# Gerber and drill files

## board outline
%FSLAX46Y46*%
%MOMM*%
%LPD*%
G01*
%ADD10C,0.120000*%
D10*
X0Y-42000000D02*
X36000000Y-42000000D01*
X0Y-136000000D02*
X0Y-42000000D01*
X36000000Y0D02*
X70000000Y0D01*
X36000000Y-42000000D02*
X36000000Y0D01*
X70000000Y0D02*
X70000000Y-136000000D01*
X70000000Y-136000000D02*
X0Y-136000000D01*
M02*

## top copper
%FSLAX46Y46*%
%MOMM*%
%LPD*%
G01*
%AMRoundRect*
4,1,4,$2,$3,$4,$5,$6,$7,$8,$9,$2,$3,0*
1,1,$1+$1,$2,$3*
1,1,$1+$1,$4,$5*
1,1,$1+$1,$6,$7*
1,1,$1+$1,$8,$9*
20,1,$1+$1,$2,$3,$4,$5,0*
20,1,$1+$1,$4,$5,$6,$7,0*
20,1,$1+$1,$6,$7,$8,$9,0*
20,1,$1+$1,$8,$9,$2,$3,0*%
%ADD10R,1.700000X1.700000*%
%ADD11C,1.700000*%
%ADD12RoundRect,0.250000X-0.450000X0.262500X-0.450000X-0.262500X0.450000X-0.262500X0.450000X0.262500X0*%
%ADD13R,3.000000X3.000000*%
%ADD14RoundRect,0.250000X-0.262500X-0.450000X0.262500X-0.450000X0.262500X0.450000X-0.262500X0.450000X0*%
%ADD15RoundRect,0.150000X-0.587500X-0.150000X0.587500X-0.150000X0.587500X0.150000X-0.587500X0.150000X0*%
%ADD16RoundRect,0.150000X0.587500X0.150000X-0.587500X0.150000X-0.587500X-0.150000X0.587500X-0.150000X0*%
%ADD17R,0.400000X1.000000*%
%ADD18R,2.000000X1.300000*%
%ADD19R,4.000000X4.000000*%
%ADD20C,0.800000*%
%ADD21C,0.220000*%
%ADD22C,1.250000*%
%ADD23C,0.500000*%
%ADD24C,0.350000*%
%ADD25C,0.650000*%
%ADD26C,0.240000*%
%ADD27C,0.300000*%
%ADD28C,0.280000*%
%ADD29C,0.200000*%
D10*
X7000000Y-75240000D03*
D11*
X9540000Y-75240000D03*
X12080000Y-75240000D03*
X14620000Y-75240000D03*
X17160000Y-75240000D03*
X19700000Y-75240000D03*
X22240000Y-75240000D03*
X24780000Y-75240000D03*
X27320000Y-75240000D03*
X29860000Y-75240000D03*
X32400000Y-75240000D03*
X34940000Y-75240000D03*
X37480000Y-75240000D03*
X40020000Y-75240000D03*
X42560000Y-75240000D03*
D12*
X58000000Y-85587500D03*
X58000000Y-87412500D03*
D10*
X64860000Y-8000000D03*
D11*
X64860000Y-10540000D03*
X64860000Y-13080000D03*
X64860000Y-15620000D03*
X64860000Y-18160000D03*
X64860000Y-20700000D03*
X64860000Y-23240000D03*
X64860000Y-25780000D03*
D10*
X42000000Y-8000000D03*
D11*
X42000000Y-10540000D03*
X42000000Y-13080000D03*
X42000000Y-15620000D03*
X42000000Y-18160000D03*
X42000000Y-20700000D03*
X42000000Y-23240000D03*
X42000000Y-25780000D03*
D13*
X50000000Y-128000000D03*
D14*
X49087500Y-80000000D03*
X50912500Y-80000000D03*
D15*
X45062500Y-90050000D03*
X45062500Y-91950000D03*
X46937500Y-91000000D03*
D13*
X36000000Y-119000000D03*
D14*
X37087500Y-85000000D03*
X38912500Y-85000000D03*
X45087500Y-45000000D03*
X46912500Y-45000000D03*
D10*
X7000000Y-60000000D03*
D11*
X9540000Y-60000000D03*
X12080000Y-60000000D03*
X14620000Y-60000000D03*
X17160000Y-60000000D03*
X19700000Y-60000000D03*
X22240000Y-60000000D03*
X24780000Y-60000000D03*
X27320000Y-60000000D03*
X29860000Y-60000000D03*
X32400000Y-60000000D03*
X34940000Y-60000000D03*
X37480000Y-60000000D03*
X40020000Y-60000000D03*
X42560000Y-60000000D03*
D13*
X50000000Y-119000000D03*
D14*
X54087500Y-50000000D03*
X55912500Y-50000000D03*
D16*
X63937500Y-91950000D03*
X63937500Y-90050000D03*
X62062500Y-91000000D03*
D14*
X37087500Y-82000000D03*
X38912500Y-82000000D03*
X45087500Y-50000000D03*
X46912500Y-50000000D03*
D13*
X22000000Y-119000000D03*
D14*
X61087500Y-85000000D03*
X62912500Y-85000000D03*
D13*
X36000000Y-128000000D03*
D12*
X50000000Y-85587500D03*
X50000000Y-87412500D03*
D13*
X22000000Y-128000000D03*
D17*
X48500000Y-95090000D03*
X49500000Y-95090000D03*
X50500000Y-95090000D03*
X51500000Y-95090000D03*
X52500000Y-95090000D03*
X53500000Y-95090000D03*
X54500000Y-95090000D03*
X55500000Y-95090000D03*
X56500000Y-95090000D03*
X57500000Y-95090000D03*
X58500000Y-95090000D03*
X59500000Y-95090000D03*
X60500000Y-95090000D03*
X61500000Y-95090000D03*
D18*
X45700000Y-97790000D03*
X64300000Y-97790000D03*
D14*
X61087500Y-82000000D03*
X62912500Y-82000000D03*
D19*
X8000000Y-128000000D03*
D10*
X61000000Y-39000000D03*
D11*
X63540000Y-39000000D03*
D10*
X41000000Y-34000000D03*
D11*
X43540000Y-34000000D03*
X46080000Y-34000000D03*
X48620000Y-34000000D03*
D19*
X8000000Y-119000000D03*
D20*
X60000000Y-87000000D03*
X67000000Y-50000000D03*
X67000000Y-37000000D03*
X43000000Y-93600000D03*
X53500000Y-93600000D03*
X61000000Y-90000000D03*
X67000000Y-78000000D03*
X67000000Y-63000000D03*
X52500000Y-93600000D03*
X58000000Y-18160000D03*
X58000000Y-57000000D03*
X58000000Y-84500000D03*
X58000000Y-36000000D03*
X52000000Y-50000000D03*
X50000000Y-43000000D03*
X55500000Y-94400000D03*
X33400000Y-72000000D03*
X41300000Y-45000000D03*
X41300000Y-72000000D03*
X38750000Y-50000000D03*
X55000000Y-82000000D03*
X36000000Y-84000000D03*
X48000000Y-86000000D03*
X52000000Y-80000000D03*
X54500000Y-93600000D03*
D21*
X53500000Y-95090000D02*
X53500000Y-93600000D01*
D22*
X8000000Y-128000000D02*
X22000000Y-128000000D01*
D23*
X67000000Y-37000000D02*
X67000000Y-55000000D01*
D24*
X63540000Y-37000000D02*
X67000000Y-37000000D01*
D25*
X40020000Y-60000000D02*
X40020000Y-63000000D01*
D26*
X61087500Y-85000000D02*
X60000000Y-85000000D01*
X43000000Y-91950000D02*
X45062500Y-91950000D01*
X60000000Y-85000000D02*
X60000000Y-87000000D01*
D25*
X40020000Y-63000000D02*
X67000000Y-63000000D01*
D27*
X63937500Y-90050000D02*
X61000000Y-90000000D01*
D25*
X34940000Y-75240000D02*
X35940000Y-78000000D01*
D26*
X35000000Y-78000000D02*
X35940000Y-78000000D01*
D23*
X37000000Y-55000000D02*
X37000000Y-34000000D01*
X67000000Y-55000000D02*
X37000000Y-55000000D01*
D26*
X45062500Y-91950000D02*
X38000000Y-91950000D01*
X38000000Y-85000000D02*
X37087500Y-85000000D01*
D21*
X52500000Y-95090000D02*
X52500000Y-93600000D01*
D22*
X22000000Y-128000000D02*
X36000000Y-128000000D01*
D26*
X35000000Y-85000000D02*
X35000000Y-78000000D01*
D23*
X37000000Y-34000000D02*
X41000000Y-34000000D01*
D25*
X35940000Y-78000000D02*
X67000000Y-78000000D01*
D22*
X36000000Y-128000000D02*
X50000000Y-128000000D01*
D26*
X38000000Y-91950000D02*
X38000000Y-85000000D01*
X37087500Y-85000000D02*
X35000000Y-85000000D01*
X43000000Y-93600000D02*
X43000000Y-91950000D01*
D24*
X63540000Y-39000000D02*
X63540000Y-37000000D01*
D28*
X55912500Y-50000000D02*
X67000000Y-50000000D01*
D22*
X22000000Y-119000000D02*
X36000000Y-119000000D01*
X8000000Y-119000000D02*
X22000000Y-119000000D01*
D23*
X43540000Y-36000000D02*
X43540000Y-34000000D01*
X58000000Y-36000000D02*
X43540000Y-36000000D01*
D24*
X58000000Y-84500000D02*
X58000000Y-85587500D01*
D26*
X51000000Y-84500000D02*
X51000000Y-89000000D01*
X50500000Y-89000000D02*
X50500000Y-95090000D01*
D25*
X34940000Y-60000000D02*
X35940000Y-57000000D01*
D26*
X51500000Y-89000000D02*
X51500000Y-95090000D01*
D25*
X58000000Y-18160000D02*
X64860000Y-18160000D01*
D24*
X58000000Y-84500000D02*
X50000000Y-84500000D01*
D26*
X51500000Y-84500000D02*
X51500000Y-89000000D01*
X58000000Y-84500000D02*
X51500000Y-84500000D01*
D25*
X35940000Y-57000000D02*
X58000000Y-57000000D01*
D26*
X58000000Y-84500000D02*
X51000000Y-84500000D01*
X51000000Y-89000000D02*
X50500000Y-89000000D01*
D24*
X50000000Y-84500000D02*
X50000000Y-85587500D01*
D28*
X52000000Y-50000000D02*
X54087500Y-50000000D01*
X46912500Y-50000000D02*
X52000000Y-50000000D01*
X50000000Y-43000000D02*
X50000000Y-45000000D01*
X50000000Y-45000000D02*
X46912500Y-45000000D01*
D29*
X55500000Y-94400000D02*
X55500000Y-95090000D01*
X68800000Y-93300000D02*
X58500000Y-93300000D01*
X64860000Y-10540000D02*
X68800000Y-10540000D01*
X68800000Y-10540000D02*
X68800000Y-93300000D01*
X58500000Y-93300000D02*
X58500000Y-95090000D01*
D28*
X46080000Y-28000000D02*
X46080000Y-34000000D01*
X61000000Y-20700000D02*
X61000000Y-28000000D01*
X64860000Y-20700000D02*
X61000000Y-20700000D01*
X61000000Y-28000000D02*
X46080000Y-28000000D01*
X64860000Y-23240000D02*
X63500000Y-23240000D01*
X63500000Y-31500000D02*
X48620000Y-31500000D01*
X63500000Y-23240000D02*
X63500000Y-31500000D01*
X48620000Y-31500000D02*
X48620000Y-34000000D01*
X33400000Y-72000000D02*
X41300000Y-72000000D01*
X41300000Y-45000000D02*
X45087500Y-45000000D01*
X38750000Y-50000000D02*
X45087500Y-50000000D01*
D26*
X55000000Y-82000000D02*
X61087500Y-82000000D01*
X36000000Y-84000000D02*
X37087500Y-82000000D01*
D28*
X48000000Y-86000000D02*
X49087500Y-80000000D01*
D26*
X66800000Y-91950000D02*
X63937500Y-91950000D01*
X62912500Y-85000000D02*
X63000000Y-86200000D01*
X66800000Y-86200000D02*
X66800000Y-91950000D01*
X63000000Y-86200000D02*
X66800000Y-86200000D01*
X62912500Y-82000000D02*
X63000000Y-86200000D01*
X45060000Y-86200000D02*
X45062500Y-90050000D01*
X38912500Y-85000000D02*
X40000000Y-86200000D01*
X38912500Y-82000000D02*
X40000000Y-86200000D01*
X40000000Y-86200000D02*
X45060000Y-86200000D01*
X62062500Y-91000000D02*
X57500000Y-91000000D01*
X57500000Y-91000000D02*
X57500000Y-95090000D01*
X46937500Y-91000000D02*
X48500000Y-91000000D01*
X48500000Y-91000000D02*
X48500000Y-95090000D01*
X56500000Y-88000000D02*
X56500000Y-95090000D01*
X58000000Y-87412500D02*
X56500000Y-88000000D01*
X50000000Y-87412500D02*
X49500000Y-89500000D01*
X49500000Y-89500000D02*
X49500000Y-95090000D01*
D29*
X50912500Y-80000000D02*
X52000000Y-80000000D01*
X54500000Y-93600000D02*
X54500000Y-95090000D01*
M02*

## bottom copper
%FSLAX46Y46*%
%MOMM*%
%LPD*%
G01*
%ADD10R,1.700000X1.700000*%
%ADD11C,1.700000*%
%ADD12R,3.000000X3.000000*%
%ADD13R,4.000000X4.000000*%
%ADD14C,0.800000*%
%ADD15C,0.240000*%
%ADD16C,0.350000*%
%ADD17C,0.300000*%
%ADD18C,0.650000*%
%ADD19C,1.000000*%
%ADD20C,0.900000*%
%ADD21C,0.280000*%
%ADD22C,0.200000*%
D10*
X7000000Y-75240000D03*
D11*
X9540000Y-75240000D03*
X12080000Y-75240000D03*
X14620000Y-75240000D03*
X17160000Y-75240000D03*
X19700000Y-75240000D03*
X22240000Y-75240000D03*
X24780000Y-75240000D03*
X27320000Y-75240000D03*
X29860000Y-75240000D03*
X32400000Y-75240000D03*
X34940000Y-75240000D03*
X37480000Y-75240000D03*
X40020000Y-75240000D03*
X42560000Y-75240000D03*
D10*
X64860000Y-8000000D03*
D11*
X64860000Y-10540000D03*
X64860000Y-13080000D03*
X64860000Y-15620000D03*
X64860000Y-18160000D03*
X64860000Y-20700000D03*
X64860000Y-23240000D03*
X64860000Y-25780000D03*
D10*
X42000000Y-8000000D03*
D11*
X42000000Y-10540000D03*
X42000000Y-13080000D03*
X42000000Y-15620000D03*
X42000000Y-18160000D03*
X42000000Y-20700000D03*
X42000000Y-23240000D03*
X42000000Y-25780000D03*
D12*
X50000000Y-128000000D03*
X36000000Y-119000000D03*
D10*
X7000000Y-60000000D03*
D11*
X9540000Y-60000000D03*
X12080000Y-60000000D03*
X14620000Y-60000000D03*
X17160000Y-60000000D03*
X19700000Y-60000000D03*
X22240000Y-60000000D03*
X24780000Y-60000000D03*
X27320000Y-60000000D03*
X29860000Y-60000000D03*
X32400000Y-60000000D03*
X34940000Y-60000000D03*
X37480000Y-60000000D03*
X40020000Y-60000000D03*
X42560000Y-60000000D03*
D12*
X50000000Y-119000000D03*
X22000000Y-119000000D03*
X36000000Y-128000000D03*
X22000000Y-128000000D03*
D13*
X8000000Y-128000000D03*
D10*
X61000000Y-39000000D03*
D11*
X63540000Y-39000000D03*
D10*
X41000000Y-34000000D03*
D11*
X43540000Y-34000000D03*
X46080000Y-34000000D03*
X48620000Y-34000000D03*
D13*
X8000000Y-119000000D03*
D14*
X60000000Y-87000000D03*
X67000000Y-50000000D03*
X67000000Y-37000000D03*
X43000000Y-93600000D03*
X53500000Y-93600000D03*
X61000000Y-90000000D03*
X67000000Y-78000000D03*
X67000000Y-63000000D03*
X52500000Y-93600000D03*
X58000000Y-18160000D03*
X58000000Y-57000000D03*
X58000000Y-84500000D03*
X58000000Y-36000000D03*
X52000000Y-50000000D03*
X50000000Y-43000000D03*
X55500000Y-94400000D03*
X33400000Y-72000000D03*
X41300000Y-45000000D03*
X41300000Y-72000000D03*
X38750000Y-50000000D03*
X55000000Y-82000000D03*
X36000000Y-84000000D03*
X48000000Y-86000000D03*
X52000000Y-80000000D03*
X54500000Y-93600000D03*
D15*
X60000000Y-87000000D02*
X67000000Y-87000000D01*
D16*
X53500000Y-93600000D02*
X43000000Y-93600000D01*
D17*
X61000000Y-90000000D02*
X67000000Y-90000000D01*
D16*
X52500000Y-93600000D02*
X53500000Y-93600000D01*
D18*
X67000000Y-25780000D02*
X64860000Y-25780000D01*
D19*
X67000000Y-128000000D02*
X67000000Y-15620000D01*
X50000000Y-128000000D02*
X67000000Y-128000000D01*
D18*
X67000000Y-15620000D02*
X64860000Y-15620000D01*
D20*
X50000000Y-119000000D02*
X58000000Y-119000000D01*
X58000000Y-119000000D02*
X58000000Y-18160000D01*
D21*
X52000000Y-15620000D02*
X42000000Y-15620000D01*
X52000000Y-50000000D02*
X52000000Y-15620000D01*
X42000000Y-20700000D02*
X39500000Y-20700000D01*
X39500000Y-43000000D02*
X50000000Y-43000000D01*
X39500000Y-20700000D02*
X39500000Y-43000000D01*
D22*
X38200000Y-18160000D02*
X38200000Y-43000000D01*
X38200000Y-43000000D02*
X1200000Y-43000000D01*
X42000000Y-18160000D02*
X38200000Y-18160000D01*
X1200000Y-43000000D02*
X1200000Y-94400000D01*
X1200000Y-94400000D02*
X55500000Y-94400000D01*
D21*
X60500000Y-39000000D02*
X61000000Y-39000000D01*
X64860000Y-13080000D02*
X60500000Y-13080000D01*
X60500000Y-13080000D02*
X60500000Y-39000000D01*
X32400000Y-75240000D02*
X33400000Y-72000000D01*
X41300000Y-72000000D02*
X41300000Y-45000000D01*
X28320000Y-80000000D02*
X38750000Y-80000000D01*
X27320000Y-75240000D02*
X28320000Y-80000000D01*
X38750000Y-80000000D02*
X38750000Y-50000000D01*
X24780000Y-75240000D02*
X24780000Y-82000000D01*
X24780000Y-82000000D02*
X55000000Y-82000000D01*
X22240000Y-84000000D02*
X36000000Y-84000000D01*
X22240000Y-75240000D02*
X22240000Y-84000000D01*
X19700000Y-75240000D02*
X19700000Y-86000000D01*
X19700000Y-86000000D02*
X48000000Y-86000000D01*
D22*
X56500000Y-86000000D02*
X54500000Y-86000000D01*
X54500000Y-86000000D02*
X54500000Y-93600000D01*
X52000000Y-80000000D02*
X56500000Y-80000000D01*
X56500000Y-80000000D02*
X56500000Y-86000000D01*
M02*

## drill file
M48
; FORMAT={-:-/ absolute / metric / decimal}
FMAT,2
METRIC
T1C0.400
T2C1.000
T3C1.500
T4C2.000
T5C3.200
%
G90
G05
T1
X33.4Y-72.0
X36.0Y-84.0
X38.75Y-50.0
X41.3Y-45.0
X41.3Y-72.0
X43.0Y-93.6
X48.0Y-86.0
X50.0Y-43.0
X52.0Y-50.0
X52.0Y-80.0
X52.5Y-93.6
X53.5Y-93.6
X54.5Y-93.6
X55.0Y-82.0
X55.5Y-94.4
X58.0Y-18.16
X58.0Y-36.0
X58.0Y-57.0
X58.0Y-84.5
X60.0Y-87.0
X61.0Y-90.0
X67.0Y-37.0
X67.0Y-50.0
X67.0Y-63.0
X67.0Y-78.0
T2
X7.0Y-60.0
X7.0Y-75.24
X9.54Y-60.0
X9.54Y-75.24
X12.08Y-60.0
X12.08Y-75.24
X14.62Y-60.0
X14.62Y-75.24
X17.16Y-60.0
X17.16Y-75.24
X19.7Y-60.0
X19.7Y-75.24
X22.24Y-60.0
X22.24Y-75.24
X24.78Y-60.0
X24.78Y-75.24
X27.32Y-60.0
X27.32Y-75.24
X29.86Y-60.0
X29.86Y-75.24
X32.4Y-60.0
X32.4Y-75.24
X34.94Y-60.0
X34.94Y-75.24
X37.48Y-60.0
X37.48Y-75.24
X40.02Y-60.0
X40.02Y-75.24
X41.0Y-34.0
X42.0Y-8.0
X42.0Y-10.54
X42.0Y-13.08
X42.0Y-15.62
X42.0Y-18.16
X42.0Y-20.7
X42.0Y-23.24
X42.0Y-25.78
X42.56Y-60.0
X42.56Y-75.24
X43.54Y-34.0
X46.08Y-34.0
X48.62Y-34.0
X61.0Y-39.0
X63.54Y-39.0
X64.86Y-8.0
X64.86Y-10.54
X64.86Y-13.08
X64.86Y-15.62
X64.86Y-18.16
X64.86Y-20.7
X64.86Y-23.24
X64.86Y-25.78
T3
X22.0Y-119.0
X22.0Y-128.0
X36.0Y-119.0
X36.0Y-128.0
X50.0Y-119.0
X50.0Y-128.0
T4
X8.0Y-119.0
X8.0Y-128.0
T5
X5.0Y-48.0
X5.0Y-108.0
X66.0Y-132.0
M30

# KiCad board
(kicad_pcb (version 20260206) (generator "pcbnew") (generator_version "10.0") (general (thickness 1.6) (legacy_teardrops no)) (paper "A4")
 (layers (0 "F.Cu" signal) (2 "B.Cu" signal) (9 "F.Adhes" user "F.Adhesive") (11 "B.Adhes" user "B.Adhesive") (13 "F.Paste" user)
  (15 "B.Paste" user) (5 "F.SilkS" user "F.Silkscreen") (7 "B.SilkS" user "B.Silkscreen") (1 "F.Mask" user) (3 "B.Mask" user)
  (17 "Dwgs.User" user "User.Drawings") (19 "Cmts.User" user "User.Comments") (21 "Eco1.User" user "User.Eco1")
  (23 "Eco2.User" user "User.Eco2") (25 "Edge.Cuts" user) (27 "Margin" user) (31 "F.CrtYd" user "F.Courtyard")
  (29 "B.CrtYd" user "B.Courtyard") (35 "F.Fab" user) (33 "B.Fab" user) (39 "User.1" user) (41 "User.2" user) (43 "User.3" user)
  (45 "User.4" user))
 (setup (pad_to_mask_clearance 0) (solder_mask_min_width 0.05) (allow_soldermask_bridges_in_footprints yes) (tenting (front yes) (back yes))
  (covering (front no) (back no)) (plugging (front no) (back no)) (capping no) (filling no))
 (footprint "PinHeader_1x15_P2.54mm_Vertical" (layer "F.Cu") (at 7 75.24 90)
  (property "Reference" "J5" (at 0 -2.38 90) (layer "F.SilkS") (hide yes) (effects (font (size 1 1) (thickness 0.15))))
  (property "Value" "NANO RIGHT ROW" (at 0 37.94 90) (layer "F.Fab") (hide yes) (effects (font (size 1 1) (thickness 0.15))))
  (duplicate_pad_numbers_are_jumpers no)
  (pad "1" thru_hole rect (at 0 0 90) (size 1.7 1.7) (drill 1) (layers "*.Cu" "*.Mask") (remove_unused_layers no))
  (pad "2" thru_hole circle (at 0 2.54 90) (size 1.7 1.7) (drill 1) (layers "*.Cu" "*.Mask") (remove_unused_layers no))
  (pad "3" thru_hole circle (at 0 5.08 90) (size 1.7 1.7) (drill 1) (layers "*.Cu" "*.Mask") (remove_unused_layers no))
  (pad "4" thru_hole circle (at 0 7.62 90) (size 1.7 1.7) (drill 1) (layers "*.Cu" "*.Mask") (remove_unused_layers no))
  (pad "5" thru_hole circle (at 0 10.16 90) (size 1.7 1.7) (drill 1) (layers "*.Cu" "*.Mask") (remove_unused_layers no)
   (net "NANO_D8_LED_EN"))
  (pad "6" thru_hole circle (at 0 12.7 90) (size 1.7 1.7) (drill 1) (layers "*.Cu" "*.Mask") (remove_unused_layers no)
   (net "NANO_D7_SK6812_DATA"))
  (pad "7" thru_hole circle (at 0 15.24 90) (size 1.7 1.7) (drill 1) (layers "*.Cu" "*.Mask") (remove_unused_layers no)
   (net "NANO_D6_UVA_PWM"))
  (pad "8" thru_hole circle (at 0 17.78 90) (size 1.7 1.7) (drill 1) (layers "*.Cu" "*.Mask") (remove_unused_layers no)
   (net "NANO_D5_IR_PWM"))
  (pad "9" thru_hole circle (at 0 20.32 90) (size 1.7 1.7) (drill 1) (layers "*.Cu" "*.Mask") (remove_unused_layers no) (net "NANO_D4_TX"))
  (pad "10" thru_hole circle (at 0 22.86 90) (size 1.7 1.7) (drill 1) (layers "*.Cu" "*.Mask") (remove_unused_layers no))
  (pad "11" thru_hole circle (at 0 25.4 90) (size 1.7 1.7) (drill 1) (layers "*.Cu" "*.Mask") (remove_unused_layers no) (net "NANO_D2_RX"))
  (pad "12" thru_hole circle (at 0 27.94 90) (size 1.7 1.7) (drill 1) (layers "*.Cu" "*.Mask") (remove_unused_layers no) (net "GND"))
  (pad "13" thru_hole circle (at 0 30.48 90) (size 1.7 1.7) (drill 1) (layers "*.Cu" "*.Mask") (remove_unused_layers no))
  (pad "14" thru_hole circle (at 0 33.02 90) (size 1.7 1.7) (drill 1) (layers "*.Cu" "*.Mask") (remove_unused_layers no))
  (pad "15" thru_hole circle (at 0 35.56 90) (size 1.7 1.7) (drill 1) (layers "*.Cu" "*.Mask") (remove_unused_layers no)))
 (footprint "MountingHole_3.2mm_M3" (layer "F.Cu") (at 5 48)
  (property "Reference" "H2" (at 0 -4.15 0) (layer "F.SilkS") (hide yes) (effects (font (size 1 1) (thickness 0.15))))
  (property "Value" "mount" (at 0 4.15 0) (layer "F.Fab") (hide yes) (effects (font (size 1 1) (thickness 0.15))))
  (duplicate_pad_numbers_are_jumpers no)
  (pad "" np_thru_hole circle (at 0 0) (size 3.2 3.2) (drill 3.2) (layers "*.Cu" "*.Mask")))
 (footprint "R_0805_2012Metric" (layer "F.Cu") (at 58 86.5 -90)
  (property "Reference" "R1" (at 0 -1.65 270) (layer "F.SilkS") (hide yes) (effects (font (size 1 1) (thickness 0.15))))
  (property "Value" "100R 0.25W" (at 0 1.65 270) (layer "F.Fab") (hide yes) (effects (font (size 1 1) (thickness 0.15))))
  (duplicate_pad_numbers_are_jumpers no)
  (pad "1" smd roundrect (at -0.9125 0 270) (size 1.025 1.4) (layers "F.Cu" "F.Mask" "F.Paste") (roundrect_rratio 0.243902) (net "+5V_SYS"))
  (pad "2" smd roundrect (at 0.9125 0 270) (size 1.025 1.4) (layers "F.Cu" "F.Mask" "F.Paste") (roundrect_rratio 0.243902) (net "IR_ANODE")))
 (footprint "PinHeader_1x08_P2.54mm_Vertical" (layer "F.Cu") (at 64.86 8)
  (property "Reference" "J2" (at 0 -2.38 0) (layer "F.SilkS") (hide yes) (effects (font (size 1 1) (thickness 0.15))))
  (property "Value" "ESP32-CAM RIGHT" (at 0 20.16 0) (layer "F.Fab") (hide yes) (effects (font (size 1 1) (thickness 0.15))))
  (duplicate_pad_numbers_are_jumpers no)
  (pad "1" thru_hole rect (at 0 0) (size 1.7 1.7) (drill 1) (layers "*.Cu" "*.Mask") (remove_unused_layers no))
  (pad "2" thru_hole circle (at 0 2.54) (size 1.7 1.7) (drill 1) (layers "*.Cu" "*.Mask") (remove_unused_layers no)
   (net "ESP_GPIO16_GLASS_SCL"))
  (pad "3" thru_hole circle (at 0 5.08) (size 1.7 1.7) (drill 1) (layers "*.Cu" "*.Mask") (remove_unused_layers no) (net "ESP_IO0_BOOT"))
  (pad "4" thru_hole circle (at 0 7.62) (size 1.7 1.7) (drill 1) (layers "*.Cu" "*.Mask") (remove_unused_layers no) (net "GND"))
  (pad "5" thru_hole circle (at 0 10.16) (size 1.7 1.7) (drill 1) (layers "*.Cu" "*.Mask") (remove_unused_layers no) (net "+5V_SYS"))
  (pad "6" thru_hole circle (at 0 12.7) (size 1.7 1.7) (drill 1) (layers "*.Cu" "*.Mask") (remove_unused_layers no) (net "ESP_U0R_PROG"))
  (pad "7" thru_hole circle (at 0 15.24) (size 1.7 1.7) (drill 1) (layers "*.Cu" "*.Mask") (remove_unused_layers no) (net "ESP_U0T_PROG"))
  (pad "8" thru_hole circle (at 0 17.78) (size 1.7 1.7) (drill 1) (layers "*.Cu" "*.Mask") (remove_unused_layers no) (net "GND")))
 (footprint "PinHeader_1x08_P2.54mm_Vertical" (layer "F.Cu") (at 42 8)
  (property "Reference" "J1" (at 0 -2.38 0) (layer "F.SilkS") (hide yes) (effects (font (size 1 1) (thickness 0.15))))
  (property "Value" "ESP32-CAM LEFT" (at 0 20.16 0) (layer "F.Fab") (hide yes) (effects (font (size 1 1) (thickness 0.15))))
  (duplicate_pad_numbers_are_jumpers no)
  (pad "1" thru_hole rect (at 0 0) (size 1.7 1.7) (drill 1) (layers "*.Cu" "*.Mask") (remove_unused_layers no))
  (pad "2" thru_hole circle (at 0 2.54) (size 1.7 1.7) (drill 1) (layers "*.Cu" "*.Mask") (remove_unused_layers no))
  (pad "3" thru_hole circle (at 0 5.08) (size 1.7 1.7) (drill 1) (layers "*.Cu" "*.Mask") (remove_unused_layers no))
  (pad "4" thru_hole circle (at 0 7.62) (size 1.7 1.7) (drill 1) (layers "*.Cu" "*.Mask") (remove_unused_layers no) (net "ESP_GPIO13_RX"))
  (pad "5" thru_hole circle (at 0 10.16) (size 1.7 1.7) (drill 1) (layers "*.Cu" "*.Mask") (remove_unused_layers no)
   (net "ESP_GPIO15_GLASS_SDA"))
  (pad "6" thru_hole circle (at 0 12.7) (size 1.7 1.7) (drill 1) (layers "*.Cu" "*.Mask") (remove_unused_layers no) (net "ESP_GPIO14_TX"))
  (pad "7" thru_hole circle (at 0 15.24) (size 1.7 1.7) (drill 1) (layers "*.Cu" "*.Mask") (remove_unused_layers no))
  (pad "8" thru_hole circle (at 0 17.78) (size 1.7 1.7) (drill 1) (layers "*.Cu" "*.Mask") (remove_unused_layers no)))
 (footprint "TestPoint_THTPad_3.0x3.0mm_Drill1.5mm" (layer "F.Cu") (at 50 128)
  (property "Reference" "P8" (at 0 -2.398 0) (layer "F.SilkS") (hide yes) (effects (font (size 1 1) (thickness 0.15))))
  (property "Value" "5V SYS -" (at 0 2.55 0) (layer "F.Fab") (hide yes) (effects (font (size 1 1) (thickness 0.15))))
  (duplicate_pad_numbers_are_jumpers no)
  (pad "1" thru_hole rect (at 0 0) (size 3 3) (drill 1.5) (layers "*.Cu" "*.Mask") (remove_unused_layers no) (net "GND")))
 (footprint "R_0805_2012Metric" (layer "F.Cu") (at 50 80)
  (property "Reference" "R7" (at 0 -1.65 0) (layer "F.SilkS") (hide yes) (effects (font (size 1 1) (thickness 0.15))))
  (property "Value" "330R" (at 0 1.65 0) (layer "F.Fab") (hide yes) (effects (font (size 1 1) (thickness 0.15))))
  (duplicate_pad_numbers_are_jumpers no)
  (pad "1" smd roundrect (at -0.9125 0) (size 1.025 1.4) (layers "F.Cu" "F.Mask" "F.Paste") (roundrect_rratio 0.243902)
   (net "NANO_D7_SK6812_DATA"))
  (pad "2" smd roundrect (at 0.9125 0) (size 1.025 1.4) (layers "F.Cu" "F.Mask" "F.Paste") (roundrect_rratio 0.243902) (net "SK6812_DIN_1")))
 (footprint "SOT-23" (layer "F.Cu") (at 46 91)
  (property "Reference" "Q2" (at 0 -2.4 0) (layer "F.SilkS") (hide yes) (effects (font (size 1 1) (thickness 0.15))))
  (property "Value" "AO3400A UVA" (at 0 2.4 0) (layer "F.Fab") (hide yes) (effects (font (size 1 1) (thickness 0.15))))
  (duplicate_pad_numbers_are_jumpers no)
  (pad "1" smd roundrect (at -0.9375 -0.95) (size 1.475 0.6) (layers "F.Cu" "F.Mask" "F.Paste") (roundrect_rratio 0.25) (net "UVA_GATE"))
  (pad "2" smd roundrect (at -0.9375 0.95) (size 1.475 0.6) (layers "F.Cu" "F.Mask" "F.Paste") (roundrect_rratio 0.25) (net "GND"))
  (pad "3" smd roundrect (at 0.9375 0) (size 1.475 0.6) (layers "F.Cu" "F.Mask" "F.Paste") (roundrect_rratio 0.25) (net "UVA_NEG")))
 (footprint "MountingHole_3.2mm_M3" (layer "F.Cu") (at 66 132)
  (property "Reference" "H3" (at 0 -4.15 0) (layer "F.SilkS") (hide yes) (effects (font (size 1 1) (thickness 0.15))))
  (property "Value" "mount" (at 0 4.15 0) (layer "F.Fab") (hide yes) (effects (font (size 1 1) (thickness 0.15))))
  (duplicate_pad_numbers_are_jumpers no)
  (pad "" np_thru_hole circle (at 0 0) (size 3.2 3.2) (drill 3.2) (layers "*.Cu" "*.Mask")))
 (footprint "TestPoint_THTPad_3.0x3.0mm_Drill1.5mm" (layer "F.Cu") (at 36 119)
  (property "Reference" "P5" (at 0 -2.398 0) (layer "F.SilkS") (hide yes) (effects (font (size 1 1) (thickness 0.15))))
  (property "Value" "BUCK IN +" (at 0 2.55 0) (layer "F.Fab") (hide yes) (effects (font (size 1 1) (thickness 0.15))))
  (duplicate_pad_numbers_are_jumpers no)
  (pad "1" thru_hole rect (at 0 0) (size 3 3) (drill 1.5) (layers "*.Cu" "*.Mask") (remove_unused_layers no) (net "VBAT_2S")))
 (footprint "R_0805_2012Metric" (layer "F.Cu") (at 38 85)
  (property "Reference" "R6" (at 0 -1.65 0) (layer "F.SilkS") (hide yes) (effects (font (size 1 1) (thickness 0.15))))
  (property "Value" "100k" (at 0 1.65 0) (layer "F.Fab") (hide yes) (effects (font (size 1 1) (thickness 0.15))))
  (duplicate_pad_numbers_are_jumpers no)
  (pad "1" smd roundrect (at -0.9125 0) (size 1.025 1.4) (layers "F.Cu" "F.Mask" "F.Paste") (roundrect_rratio 0.243902) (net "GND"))
  (pad "2" smd roundrect (at 0.9125 0) (size 1.025 1.4) (layers "F.Cu" "F.Mask" "F.Paste") (roundrect_rratio 0.243902) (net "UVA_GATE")))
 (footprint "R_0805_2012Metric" (layer "F.Cu") (at 46 45)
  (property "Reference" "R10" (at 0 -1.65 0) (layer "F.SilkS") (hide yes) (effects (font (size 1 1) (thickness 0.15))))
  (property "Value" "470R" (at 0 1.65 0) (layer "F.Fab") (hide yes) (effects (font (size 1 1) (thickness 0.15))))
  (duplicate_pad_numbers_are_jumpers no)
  (pad "1" smd roundrect (at -0.9125 0) (size 1.025 1.4) (layers "F.Cu" "F.Mask" "F.Paste") (roundrect_rratio 0.243902) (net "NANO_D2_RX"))
  (pad "2" smd roundrect (at 0.9125 0) (size 1.025 1.4) (layers "F.Cu" "F.Mask" "F.Paste") (roundrect_rratio 0.243902) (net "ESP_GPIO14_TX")))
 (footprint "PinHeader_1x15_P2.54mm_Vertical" (layer "F.Cu") (at 7 60 90)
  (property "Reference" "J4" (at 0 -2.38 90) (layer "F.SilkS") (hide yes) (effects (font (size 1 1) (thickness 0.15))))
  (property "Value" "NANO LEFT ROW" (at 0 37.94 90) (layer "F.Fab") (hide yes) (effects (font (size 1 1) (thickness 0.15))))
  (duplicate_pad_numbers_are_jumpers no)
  (pad "1" thru_hole rect (at 0 0 90) (size 1.7 1.7) (drill 1) (layers "*.Cu" "*.Mask") (remove_unused_layers no))
  (pad "2" thru_hole circle (at 0 2.54 90) (size 1.7 1.7) (drill 1) (layers "*.Cu" "*.Mask") (remove_unused_layers no))
  (pad "3" thru_hole circle (at 0 5.08 90) (size 1.7 1.7) (drill 1) (layers "*.Cu" "*.Mask") (remove_unused_layers no))
  (pad "4" thru_hole circle (at 0 7.62 90) (size 1.7 1.7) (drill 1) (layers "*.Cu" "*.Mask") (remove_unused_layers no))
  (pad "5" thru_hole circle (at 0 10.16 90) (size 1.7 1.7) (drill 1) (layers "*.Cu" "*.Mask") (remove_unused_layers no))
  (pad "6" thru_hole circle (at 0 12.7 90) (size 1.7 1.7) (drill 1) (layers "*.Cu" "*.Mask") (remove_unused_layers no))
  (pad "7" thru_hole circle (at 0 15.24 90) (size 1.7 1.7) (drill 1) (layers "*.Cu" "*.Mask") (remove_unused_layers no))
  (pad "8" thru_hole circle (at 0 17.78 90) (size 1.7 1.7) (drill 1) (layers "*.Cu" "*.Mask") (remove_unused_layers no))
  (pad "9" thru_hole circle (at 0 20.32 90) (size 1.7 1.7) (drill 1) (layers "*.Cu" "*.Mask") (remove_unused_layers no))
  (pad "10" thru_hole circle (at 0 22.86 90) (size 1.7 1.7) (drill 1) (layers "*.Cu" "*.Mask") (remove_unused_layers no))
  (pad "11" thru_hole circle (at 0 25.4 90) (size 1.7 1.7) (drill 1) (layers "*.Cu" "*.Mask") (remove_unused_layers no))
  (pad "12" thru_hole circle (at 0 27.94 90) (size 1.7 1.7) (drill 1) (layers "*.Cu" "*.Mask") (remove_unused_layers no) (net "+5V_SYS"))
  (pad "13" thru_hole circle (at 0 30.48 90) (size 1.7 1.7) (drill 1) (layers "*.Cu" "*.Mask") (remove_unused_layers no))
  (pad "14" thru_hole circle (at 0 33.02 90) (size 1.7 1.7) (drill 1) (layers "*.Cu" "*.Mask") (remove_unused_layers no) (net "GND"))
  (pad "15" thru_hole circle (at 0 35.56 90) (size 1.7 1.7) (drill 1) (layers "*.Cu" "*.Mask") (remove_unused_layers no)))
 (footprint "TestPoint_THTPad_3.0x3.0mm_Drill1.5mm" (layer "F.Cu") (at 50 119)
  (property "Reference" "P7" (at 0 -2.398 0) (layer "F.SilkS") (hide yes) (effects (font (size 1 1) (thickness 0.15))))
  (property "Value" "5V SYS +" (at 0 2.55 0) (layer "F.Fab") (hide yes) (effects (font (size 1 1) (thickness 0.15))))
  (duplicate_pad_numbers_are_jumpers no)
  (pad "1" thru_hole rect (at 0 0) (size 3 3) (drill 1.5) (layers "*.Cu" "*.Mask") (remove_unused_layers no) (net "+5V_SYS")))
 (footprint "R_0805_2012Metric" (layer "F.Cu") (at 55 50)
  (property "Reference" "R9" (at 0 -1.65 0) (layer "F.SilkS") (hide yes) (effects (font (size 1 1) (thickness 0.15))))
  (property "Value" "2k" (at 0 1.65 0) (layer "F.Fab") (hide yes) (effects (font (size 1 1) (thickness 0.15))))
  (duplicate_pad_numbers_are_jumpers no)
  (pad "1" smd roundrect (at -0.9125 0) (size 1.025 1.4) (layers "F.Cu" "F.Mask" "F.Paste") (roundrect_rratio 0.243902)
   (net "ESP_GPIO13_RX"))
  (pad "2" smd roundrect (at 0.9125 0) (size 1.025 1.4) (layers "F.Cu" "F.Mask" "F.Paste") (roundrect_rratio 0.243902) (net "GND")))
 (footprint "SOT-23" (layer "F.Cu") (at 63 91 180)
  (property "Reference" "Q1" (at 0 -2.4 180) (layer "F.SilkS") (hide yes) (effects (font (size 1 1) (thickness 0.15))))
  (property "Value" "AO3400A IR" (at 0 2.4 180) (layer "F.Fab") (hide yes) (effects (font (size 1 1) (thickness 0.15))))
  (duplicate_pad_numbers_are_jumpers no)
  (pad "1" smd roundrect (at -0.9375 -0.95 180) (size 1.475 0.6) (layers "F.Cu" "F.Mask" "F.Paste") (roundrect_rratio 0.25) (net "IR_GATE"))
  (pad "2" smd roundrect (at -0.9375 0.95 180) (size 1.475 0.6) (layers "F.Cu" "F.Mask" "F.Paste") (roundrect_rratio 0.25) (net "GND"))
  (pad "3" smd roundrect (at 0.9375 0 180) (size 1.475 0.6) (layers "F.Cu" "F.Mask" "F.Paste") (roundrect_rratio 0.25) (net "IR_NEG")))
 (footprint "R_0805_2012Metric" (layer "F.Cu") (at 38 82)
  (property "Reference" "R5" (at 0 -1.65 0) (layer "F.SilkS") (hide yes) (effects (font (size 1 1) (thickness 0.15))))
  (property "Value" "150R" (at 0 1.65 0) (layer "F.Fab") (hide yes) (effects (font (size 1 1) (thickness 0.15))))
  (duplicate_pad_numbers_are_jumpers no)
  (pad "1" smd roundrect (at -0.9125 0) (size 1.025 1.4) (layers "F.Cu" "F.Mask" "F.Paste") (roundrect_rratio 0.243902)
   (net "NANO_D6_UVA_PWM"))
  (pad "2" smd roundrect (at 0.9125 0) (size 1.025 1.4) (layers "F.Cu" "F.Mask" "F.Paste") (roundrect_rratio 0.243902) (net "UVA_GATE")))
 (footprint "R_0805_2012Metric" (layer "F.Cu") (at 46 50)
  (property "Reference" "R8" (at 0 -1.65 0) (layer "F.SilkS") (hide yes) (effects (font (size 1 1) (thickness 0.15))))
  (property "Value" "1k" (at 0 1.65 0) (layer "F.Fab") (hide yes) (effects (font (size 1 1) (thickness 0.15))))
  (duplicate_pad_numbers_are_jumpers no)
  (pad "1" smd roundrect (at -0.9125 0) (size 1.025 1.4) (layers "F.Cu" "F.Mask" "F.Paste") (roundrect_rratio 0.243902) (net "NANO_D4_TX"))
  (pad "2" smd roundrect (at 0.9125 0) (size 1.025 1.4) (layers "F.Cu" "F.Mask" "F.Paste") (roundrect_rratio 0.243902) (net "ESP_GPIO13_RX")))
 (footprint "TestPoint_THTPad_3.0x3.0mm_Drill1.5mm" (layer "F.Cu") (at 22 119)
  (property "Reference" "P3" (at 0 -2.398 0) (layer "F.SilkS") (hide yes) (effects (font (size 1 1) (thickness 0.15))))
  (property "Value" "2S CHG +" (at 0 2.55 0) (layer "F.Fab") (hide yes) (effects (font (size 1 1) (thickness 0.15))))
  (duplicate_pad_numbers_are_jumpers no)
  (pad "1" thru_hole rect (at 0 0) (size 3 3) (drill 1.5) (layers "*.Cu" "*.Mask") (remove_unused_layers no) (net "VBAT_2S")))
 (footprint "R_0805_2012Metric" (layer "F.Cu") (at 62 85)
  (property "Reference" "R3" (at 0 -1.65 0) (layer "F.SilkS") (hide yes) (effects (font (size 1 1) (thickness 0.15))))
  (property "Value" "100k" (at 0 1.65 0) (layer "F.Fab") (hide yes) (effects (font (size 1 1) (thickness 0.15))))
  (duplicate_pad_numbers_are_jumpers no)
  (pad "1" smd roundrect (at -0.9125 0) (size 1.025 1.4) (layers "F.Cu" "F.Mask" "F.Paste") (roundrect_rratio 0.243902) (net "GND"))
  (pad "2" smd roundrect (at 0.9125 0) (size 1.025 1.4) (layers "F.Cu" "F.Mask" "F.Paste") (roundrect_rratio 0.243902) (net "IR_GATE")))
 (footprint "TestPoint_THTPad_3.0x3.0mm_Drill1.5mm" (layer "F.Cu") (at 36 128)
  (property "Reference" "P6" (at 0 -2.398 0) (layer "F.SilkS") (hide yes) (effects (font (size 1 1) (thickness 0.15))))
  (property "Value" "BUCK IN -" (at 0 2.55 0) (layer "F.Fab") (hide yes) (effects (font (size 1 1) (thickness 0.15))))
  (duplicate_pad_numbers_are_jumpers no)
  (pad "1" thru_hole rect (at 0 0) (size 3 3) (drill 1.5) (layers "*.Cu" "*.Mask") (remove_unused_layers no) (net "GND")))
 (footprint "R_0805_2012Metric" (layer "F.Cu") (at 50 86.5 -90)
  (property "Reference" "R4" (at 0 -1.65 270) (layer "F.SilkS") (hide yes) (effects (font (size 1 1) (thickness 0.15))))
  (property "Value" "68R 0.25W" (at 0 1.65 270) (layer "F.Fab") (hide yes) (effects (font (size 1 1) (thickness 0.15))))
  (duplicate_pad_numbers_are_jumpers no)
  (pad "1" smd roundrect (at -0.9125 0 270) (size 1.025 1.4) (layers "F.Cu" "F.Mask" "F.Paste") (roundrect_rratio 0.243902) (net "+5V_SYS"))
  (pad "2" smd roundrect (at 0.9125 0 270) (size 1.025 1.4) (layers "F.Cu" "F.Mask" "F.Paste") (roundrect_rratio 0.243902) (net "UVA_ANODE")))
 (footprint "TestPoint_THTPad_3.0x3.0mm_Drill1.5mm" (layer "F.Cu") (at 22 128)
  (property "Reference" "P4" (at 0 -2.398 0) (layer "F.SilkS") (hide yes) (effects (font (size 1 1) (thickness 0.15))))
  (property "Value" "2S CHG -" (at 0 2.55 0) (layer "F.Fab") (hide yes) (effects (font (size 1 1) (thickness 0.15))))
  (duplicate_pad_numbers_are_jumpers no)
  (pad "1" thru_hole rect (at 0 0) (size 3 3) (drill 1.5) (layers "*.Cu" "*.Mask") (remove_unused_layers no) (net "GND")))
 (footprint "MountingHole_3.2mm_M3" (layer "F.Cu") (at 5 108)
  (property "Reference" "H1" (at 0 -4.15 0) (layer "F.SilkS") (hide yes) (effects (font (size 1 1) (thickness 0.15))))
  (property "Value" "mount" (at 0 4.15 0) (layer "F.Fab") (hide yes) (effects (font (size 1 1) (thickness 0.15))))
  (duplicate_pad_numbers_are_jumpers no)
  (pad "" np_thru_hole circle (at 0 0) (size 3.2 3.2) (drill 3.2) (layers "*.Cu" "*.Mask")))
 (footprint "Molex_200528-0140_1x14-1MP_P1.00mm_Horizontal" (layer "F.Cu") (at 55 96)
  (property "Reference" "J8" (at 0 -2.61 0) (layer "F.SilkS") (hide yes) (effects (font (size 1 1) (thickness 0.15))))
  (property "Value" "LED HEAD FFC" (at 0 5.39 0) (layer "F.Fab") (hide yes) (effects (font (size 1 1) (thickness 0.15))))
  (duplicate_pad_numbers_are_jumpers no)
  (pad "1" smd rect (at -6.5 -0.91) (size 0.4 1) (layers "F.Cu" "F.Mask" "F.Paste") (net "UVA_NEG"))
  (pad "2" smd rect (at -5.5 -0.91) (size 0.4 1) (layers "F.Cu" "F.Mask" "F.Paste") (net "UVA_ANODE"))
  (pad "3" smd rect (at -4.5 -0.91) (size 0.4 1) (layers "F.Cu" "F.Mask" "F.Paste") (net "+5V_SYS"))
  (pad "4" smd rect (at -3.5 -0.91) (size 0.4 1) (layers "F.Cu" "F.Mask" "F.Paste") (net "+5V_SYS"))
  (pad "5" smd rect (at -2.5 -0.91) (size 0.4 1) (layers "F.Cu" "F.Mask" "F.Paste") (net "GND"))
  (pad "6" smd rect (at -1.5 -0.91) (size 0.4 1) (layers "F.Cu" "F.Mask" "F.Paste") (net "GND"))
  (pad "7" smd rect (at -0.5 -0.91) (size 0.4 1) (layers "F.Cu" "F.Mask" "F.Paste") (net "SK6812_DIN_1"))
  (pad "8" smd rect (at 0.5 -0.91) (size 0.4 1) (layers "F.Cu" "F.Mask" "F.Paste") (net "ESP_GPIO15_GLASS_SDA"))
  (pad "9" smd rect (at 1.5 -0.91) (size 0.4 1) (layers "F.Cu" "F.Mask" "F.Paste") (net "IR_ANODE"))
  (pad "10" smd rect (at 2.5 -0.91) (size 0.4 1) (layers "F.Cu" "F.Mask" "F.Paste") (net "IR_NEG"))
  (pad "11" smd rect (at 3.5 -0.91) (size 0.4 1) (layers "F.Cu" "F.Mask" "F.Paste") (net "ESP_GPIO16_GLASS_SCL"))
  (pad "12" smd rect (at 4.5 -0.91) (size 0.4 1) (layers "F.Cu" "F.Mask" "F.Paste"))
  (pad "13" smd rect (at 5.5 -0.91) (size 0.4 1) (layers "F.Cu" "F.Mask" "F.Paste"))
  (pad "14" smd rect (at 6.5 -0.91) (size 0.4 1) (layers "F.Cu" "F.Mask" "F.Paste"))
  (pad "MP" smd rect (at -9.3 1.79) (size 2 1.3) (layers "F.Cu" "F.Mask" "F.Paste"))
  (pad "MP" smd rect (at 9.3 1.79) (size 2 1.3) (layers "F.Cu" "F.Mask" "F.Paste")))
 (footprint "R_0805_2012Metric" (layer "F.Cu") (at 62 82)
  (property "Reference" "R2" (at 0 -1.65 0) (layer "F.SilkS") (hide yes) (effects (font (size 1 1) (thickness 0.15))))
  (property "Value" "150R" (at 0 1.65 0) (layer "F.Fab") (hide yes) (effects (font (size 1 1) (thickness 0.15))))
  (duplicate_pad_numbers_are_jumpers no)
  (pad "1" smd roundrect (at -0.9125 0) (size 1.025 1.4) (layers "F.Cu" "F.Mask" "F.Paste") (roundrect_rratio 0.243902)
   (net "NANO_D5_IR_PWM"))
  (pad "2" smd roundrect (at 0.9125 0) (size 1.025 1.4) (layers "F.Cu" "F.Mask" "F.Paste") (roundrect_rratio 0.243902) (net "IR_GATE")))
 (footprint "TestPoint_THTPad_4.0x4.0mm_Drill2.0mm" (layer "F.Cu") (at 8 128)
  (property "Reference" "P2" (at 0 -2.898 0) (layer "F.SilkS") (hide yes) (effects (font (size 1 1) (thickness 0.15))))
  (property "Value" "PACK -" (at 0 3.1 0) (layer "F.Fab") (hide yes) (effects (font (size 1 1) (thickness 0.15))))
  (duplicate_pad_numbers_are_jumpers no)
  (pad "1" thru_hole rect (at 0 0) (size 4 4) (drill 2) (layers "*.Cu" "*.Mask") (remove_unused_layers no) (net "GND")))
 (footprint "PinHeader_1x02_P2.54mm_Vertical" (layer "F.Cu") (at 61 39 90)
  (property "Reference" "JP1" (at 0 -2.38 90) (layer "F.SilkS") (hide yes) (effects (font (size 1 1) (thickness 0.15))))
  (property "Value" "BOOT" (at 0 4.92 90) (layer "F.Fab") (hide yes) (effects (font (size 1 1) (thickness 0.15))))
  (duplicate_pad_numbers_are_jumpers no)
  (pad "1" thru_hole rect (at 0 0 90) (size 1.7 1.7) (drill 1) (layers "*.Cu" "*.Mask") (remove_unused_layers no) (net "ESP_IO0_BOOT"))
  (pad "2" thru_hole circle (at 0 2.54 90) (size 1.7 1.7) (drill 1) (layers "*.Cu" "*.Mask") (remove_unused_layers no) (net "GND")))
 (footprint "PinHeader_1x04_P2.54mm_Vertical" (layer "F.Cu") (at 41 34 90)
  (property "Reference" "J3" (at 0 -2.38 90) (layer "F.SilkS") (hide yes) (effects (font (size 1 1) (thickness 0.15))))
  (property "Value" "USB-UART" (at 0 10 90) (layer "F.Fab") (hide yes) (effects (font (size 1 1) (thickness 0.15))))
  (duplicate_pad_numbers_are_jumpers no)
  (pad "1" thru_hole rect (at 0 0 90) (size 1.7 1.7) (drill 1) (layers "*.Cu" "*.Mask") (remove_unused_layers no) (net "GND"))
  (pad "2" thru_hole circle (at 0 2.54 90) (size 1.7 1.7) (drill 1) (layers "*.Cu" "*.Mask") (remove_unused_layers no) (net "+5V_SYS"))
  (pad "3" thru_hole circle (at 0 5.08 90) (size 1.7 1.7) (drill 1) (layers "*.Cu" "*.Mask") (remove_unused_layers no) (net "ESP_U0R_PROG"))
  (pad "4" thru_hole circle (at 0 7.62 90) (size 1.7 1.7) (drill 1) (layers "*.Cu" "*.Mask") (remove_unused_layers no) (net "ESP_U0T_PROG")))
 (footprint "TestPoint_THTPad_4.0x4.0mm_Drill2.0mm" (layer "F.Cu") (at 8 119)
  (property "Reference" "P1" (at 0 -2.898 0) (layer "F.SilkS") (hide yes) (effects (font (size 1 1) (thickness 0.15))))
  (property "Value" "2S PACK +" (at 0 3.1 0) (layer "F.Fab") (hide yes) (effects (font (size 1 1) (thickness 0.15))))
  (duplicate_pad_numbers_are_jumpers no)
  (pad "1" thru_hole rect (at 0 0) (size 4 4) (drill 2) (layers "*.Cu" "*.Mask") (remove_unused_layers no) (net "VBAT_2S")))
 (gr_line (start 0 42) (end 36 42) (stroke (width 0.12) (type default)) (layer "Edge.Cuts"))
 (gr_line (start 0 136) (end 0 42) (stroke (width 0.12) (type default)) (layer "Edge.Cuts"))
 (gr_line (start 36 0) (end 70 0) (stroke (width 0.12) (type default)) (layer "Edge.Cuts"))
 (gr_line (start 36 42) (end 36 0) (stroke (width 0.12) (type default)) (layer "Edge.Cuts"))
 (gr_line (start 70 0) (end 70 136) (stroke (width 0.12) (type default)) (layer "Edge.Cuts"))
 (gr_line (start 70 136) (end 0 136) (stroke (width 0.12) (type default)) (layer "Edge.Cuts"))
 (segment (start 53.5 95.09) (end 53.5 93.6) (width 0.22) (layer "F.Cu") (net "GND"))
 (segment (start 8 128) (end 22 128) (width 1.25) (layer "F.Cu") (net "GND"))
 (segment (start 67 37) (end 67 55) (width 0.5) (layer "F.Cu") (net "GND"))
 (segment (start 63.54 37) (end 67 37) (width 0.35) (layer "F.Cu") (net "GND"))
 (segment (start 40.02 60) (end 40.02 63) (width 0.65) (layer "F.Cu") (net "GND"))
 (segment (start 61.0875 85) (end 60 85) (width 0.24) (layer "F.Cu") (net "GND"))
 (segment (start 43 91.95) (end 45.0625 91.95) (width 0.24) (layer "F.Cu") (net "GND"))
 (segment (start 60 85) (end 60 87) (width 0.24) (layer "F.Cu") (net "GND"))
 (segment (start 40.02 63) (end 67 63) (width 0.65) (layer "F.Cu") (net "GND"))
 (segment (start 63.9375 90.05) (end 61 90) (width 0.3) (layer "F.Cu") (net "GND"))
 (segment (start 34.94 75.24) (end 35.94 78) (width 0.65) (layer "F.Cu") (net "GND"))
 (segment (start 35 78) (end 35.94 78) (width 0.24) (layer "F.Cu") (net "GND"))
 (segment (start 37 55) (end 37 34) (width 0.5) (layer "F.Cu") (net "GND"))
 (segment (start 67 55) (end 37 55) (width 0.5) (layer "F.Cu") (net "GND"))
 (segment (start 45.0625 91.95) (end 38 91.95) (width 0.24) (layer "F.Cu") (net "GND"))
 (segment (start 38 85) (end 37.0875 85) (width 0.24) (layer "F.Cu") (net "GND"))
 (segment (start 52.5 95.09) (end 52.5 93.6) (width 0.22) (layer "F.Cu") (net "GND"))
 (segment (start 22 128) (end 36 128) (width 1.25) (layer "F.Cu") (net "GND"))
 (segment (start 35 85) (end 35 78) (width 0.24) (layer "F.Cu") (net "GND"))
 (segment (start 37 34) (end 41 34) (width 0.5) (layer "F.Cu") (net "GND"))
 (segment (start 35.94 78) (end 67 78) (width 0.65) (layer "F.Cu") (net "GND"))
 (segment (start 36 128) (end 50 128) (width 1.25) (layer "F.Cu") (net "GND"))
 (segment (start 38 91.95) (end 38 85) (width 0.24) (layer "F.Cu") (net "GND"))
 (segment (start 37.0875 85) (end 35 85) (width 0.24) (layer "F.Cu") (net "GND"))
 (segment (start 43 93.6) (end 43 91.95) (width 0.24) (layer "F.Cu") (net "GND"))
 (segment (start 63.54 39) (end 63.54 37) (width 0.35) (layer "F.Cu") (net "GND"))
 (segment (start 55.9125 50) (end 67 50) (width 0.28) (layer "F.Cu") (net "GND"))
 (via (at 60 87) (size 0.8) (drill 0.4) (layers "F.Cu" "B.Cu") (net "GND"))
 (via (at 67 50) (size 0.8) (drill 0.4) (layers "F.Cu" "B.Cu") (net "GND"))
 (via (at 67 37) (size 0.8) (drill 0.4) (layers "F.Cu" "B.Cu") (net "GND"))
 (via (at 43 93.6) (size 0.8) (drill 0.4) (layers "F.Cu" "B.Cu") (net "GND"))
 (via (at 53.5 93.6) (size 0.8) (drill 0.4) (layers "F.Cu" "B.Cu") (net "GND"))
 (via (at 61 90) (size 0.8) (drill 0.4) (layers "F.Cu" "B.Cu") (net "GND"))
 (via (at 67 78) (size 0.8) (drill 0.4) (layers "F.Cu" "B.Cu") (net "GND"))
 (via (at 67 63) (size 0.8) (drill 0.4) (layers "F.Cu" "B.Cu") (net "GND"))
 (via (at 52.5 93.6) (size 0.8) (drill 0.4) (layers "F.Cu" "B.Cu") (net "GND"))
 (segment (start 60 87) (end 67 87) (width 0.24) (layer "B.Cu") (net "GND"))
 (segment (start 53.5 93.6) (end 43 93.6) (width 0.35) (layer "B.Cu") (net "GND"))
 (segment (start 61 90) (end 67 90) (width 0.3) (layer "B.Cu") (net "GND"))
 (segment (start 52.5 93.6) (end 53.5 93.6) (width 0.35) (layer "B.Cu") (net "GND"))
 (segment (start 67 25.78) (end 64.86 25.78) (width 0.65) (layer "B.Cu") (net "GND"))
 (segment (start 67 128) (end 67 15.62) (width 1) (layer "B.Cu") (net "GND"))
 (segment (start 50 128) (end 67 128) (width 1) (layer "B.Cu") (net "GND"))
 (segment (start 67 15.62) (end 64.86 15.62) (width 0.65) (layer "B.Cu") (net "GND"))
 (segment (start 22 119) (end 36 119) (width 1.25) (layer "F.Cu") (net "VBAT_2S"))
 (segment (start 8 119) (end 22 119) (width 1.25) (layer "F.Cu") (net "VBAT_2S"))
 (segment (start 43.54 36) (end 43.54 34) (width 0.5) (layer "F.Cu") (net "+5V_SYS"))
 (segment (start 58 36) (end 43.54 36) (width 0.5) (layer "F.Cu") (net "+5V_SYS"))
 (segment (start 58 84.5) (end 58 85.5875) (width 0.35) (layer "F.Cu") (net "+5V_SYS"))
 (segment (start 51 84.5) (end 51 89) (width 0.24) (layer "F.Cu") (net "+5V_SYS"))
 (segment (start 50.5 89) (end 50.5 95.09) (width 0.24) (layer "F.Cu") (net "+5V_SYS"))
 (segment (start 34.94 60) (end 35.94 57) (width 0.65) (layer "F.Cu") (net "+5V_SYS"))
 (segment (start 51.5 89) (end 51.5 95.09) (width 0.24) (layer "F.Cu") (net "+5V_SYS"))
 (segment (start 58 18.16) (end 64.86 18.16) (width 0.65) (layer "F.Cu") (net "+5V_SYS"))
 (segment (start 58 84.5) (end 50 84.5) (width 0.35) (layer "F.Cu") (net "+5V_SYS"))
 (segment (start 51.5 84.5) (end 51.5 89) (width 0.24) (layer "F.Cu") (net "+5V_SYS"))
 (segment (start 58 84.5) (end 51.5 84.5) (width 0.24) (layer "F.Cu") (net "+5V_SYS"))
 (segment (start 35.94 57) (end 58 57) (width 0.65) (layer "F.Cu") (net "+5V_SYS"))
 (segment (start 58 84.5) (end 51 84.5) (width 0.24) (layer "F.Cu") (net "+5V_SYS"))
 (segment (start 51 89) (end 50.5 89) (width 0.24) (layer "F.Cu") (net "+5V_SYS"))
 (segment (start 50 84.5) (end 50 85.5875) (width 0.35) (layer "F.Cu") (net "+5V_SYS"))
 (via (at 58 18.16) (size 0.8) (drill 0.4) (layers "F.Cu" "B.Cu") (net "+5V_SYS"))
 (via (at 58 57) (size 0.8) (drill 0.4) (layers "F.Cu" "B.Cu") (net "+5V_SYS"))
 (via (at 58 84.5) (size 0.8) (drill 0.4) (layers "F.Cu" "B.Cu") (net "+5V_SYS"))
 (via (at 58 36) (size 0.8) (drill 0.4) (layers "F.Cu" "B.Cu") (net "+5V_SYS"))
 (segment (start 50 119) (end 58 119) (width 0.9) (layer "B.Cu") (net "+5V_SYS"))
 (segment (start 58 119) (end 58 18.16) (width 0.9) (layer "B.Cu") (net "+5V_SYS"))
 (segment (start 52 50) (end 54.0875 50) (width 0.28) (layer "F.Cu") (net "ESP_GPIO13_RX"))
 (segment (start 46.9125 50) (end 52 50) (width 0.28) (layer "F.Cu") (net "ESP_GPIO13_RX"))
 (via (at 52 50) (size 0.8) (drill 0.4) (layers "F.Cu" "B.Cu") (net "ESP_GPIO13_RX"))
 (segment (start 52 15.62) (end 42 15.62) (width 0.28) (layer "B.Cu") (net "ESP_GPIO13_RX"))
 (segment (start 52 50) (end 52 15.62) (width 0.28) (layer "B.Cu") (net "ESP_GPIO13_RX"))
 (segment (start 50 43) (end 50 45) (width 0.28) (layer "F.Cu") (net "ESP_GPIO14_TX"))
 (segment (start 50 45) (end 46.9125 45) (width 0.28) (layer "F.Cu") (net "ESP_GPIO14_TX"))
 (via (at 50 43) (size 0.8) (drill 0.4) (layers "F.Cu" "B.Cu") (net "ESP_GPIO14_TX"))
 (segment (start 42 20.7) (end 39.5 20.7) (width 0.28) (layer "B.Cu") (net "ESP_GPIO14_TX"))
 (segment (start 39.5 43) (end 50 43) (width 0.28) (layer "B.Cu") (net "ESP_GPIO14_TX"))
 (segment (start 39.5 20.7) (end 39.5 43) (width 0.28) (layer "B.Cu") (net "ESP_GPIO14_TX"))
 (segment (start 55.5 94.4) (end 55.5 95.09) (width 0.2) (layer "F.Cu") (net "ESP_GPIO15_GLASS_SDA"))
 (via (at 55.5 94.4) (size 0.8) (drill 0.4) (layers "F.Cu" "B.Cu") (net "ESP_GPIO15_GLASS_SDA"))
 (segment (start 38.2 18.16) (end 38.2 43) (width 0.2) (layer "B.Cu") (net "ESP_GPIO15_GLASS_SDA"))
 (segment (start 38.2 43) (end 1.2 43) (width 0.2) (layer "B.Cu") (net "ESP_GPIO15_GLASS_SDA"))
 (segment (start 42 18.16) (end 38.2 18.16) (width 0.2) (layer "B.Cu") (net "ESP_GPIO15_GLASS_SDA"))
 (segment (start 1.2 43) (end 1.2 94.4) (width 0.2) (layer "B.Cu") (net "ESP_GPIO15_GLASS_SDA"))
 (segment (start 1.2 94.4) (end 55.5 94.4) (width 0.2) (layer "B.Cu") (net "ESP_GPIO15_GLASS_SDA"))
 (segment (start 68.8 93.3) (end 58.5 93.3) (width 0.2) (layer "F.Cu") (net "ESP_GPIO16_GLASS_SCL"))
 (segment (start 64.86 10.54) (end 68.8 10.54) (width 0.2) (layer "F.Cu") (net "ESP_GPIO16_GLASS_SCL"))
 (segment (start 68.8 10.54) (end 68.8 93.3) (width 0.2) (layer "F.Cu") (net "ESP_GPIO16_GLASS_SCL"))
 (segment (start 58.5 93.3) (end 58.5 95.09) (width 0.2) (layer "F.Cu") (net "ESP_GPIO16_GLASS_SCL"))
 (segment (start 46.08 28) (end 46.08 34) (width 0.28) (layer "F.Cu") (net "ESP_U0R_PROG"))
 (segment (start 61 20.7) (end 61 28) (width 0.28) (layer "F.Cu") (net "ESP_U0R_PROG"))
 (segment (start 64.86 20.7) (end 61 20.7) (width 0.28) (layer "F.Cu") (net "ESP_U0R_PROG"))
 (segment (start 61 28) (end 46.08 28) (width 0.28) (layer "F.Cu") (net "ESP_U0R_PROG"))
 (segment (start 64.86 23.24) (end 63.5 23.24) (width 0.28) (layer "F.Cu") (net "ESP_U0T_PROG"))
 (segment (start 63.5 31.5) (end 48.62 31.5) (width 0.28) (layer "F.Cu") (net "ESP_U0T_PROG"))
 (segment (start 63.5 23.24) (end 63.5 31.5) (width 0.28) (layer "F.Cu") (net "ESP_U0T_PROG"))
 (segment (start 48.62 31.5) (end 48.62 34) (width 0.28) (layer "F.Cu") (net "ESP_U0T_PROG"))
 (segment (start 60.5 39) (end 61 39) (width 0.28) (layer "B.Cu") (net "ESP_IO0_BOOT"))
 (segment (start 64.86 13.08) (end 60.5 13.08) (width 0.28) (layer "B.Cu") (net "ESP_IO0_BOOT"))
 (segment (start 60.5 13.08) (end 60.5 39) (width 0.28) (layer "B.Cu") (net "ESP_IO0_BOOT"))
 (segment (start 33.4 72) (end 41.3 72) (width 0.28) (layer "F.Cu") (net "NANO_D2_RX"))
 (segment (start 41.3 45) (end 45.0875 45) (width 0.28) (layer "F.Cu") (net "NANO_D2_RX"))
 (via (at 33.4 72) (size 0.8) (drill 0.4) (layers "F.Cu" "B.Cu") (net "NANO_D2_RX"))
 (via (at 41.3 45) (size 0.8) (drill 0.4) (layers "F.Cu" "B.Cu") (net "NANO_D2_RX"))
 (via (at 41.3 72) (size 0.8) (drill 0.4) (layers "F.Cu" "B.Cu") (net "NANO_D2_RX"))
 (segment (start 32.4 75.24) (end 33.4 72) (width 0.28) (layer "B.Cu") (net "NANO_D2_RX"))
 (segment (start 41.3 72) (end 41.3 45) (width 0.28) (layer "B.Cu") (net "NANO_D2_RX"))
 (segment (start 38.75 50) (end 45.0875 50) (width 0.28) (layer "F.Cu") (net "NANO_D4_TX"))
 (via (at 38.75 50) (size 0.8) (drill 0.4) (layers "F.Cu" "B.Cu") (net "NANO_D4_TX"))
 (segment (start 28.32 80) (end 38.75 80) (width 0.28) (layer "B.Cu") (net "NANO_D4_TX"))
 (segment (start 27.32 75.24) (end 28.32 80) (width 0.28) (layer "B.Cu") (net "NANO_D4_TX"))
 (segment (start 38.75 80) (end 38.75 50) (width 0.28) (layer "B.Cu") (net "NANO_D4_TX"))
 (segment (start 55 82) (end 61.0875 82) (width 0.24) (layer "F.Cu") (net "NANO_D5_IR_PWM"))
 (via (at 55 82) (size 0.8) (drill 0.4) (layers "F.Cu" "B.Cu") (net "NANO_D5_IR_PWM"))
 (segment (start 24.78 75.24) (end 24.78 82) (width 0.28) (layer "B.Cu") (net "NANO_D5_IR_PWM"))
 (segment (start 24.78 82) (end 55 82) (width 0.28) (layer "B.Cu") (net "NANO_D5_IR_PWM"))
 (segment (start 36 84) (end 37.0875 82) (width 0.24) (layer "F.Cu") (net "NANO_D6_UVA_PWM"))
 (via (at 36 84) (size 0.8) (drill 0.4) (layers "F.Cu" "B.Cu") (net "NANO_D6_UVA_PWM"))
 (segment (start 22.24 84) (end 36 84) (width 0.28) (layer "B.Cu") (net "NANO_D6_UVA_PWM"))
 (segment (start 22.24 75.24) (end 22.24 84) (width 0.28) (layer "B.Cu") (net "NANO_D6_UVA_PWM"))
 (segment (start 48 86) (end 49.0875 80) (width 0.28) (layer "F.Cu") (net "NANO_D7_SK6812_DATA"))
 (via (at 48 86) (size 0.8) (drill 0.4) (layers "F.Cu" "B.Cu") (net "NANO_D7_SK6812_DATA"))
 (segment (start 19.7 75.24) (end 19.7 86) (width 0.28) (layer "B.Cu") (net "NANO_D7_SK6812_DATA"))
 (segment (start 19.7 86) (end 48 86) (width 0.28) (layer "B.Cu") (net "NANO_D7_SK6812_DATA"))
 (segment (start 66.8 91.95) (end 63.9375 91.95) (width 0.24) (layer "F.Cu") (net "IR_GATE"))
 (segment (start 62.9125 85) (end 63 86.2) (width 0.24) (layer "F.Cu") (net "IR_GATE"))
 (segment (start 66.8 86.2) (end 66.8 91.95) (width 0.24) (layer "F.Cu") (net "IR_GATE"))
 (segment (start 63 86.2) (end 66.8 86.2) (width 0.24) (layer "F.Cu") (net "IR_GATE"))
 (segment (start 62.9125 82) (end 63 86.2) (width 0.24) (layer "F.Cu") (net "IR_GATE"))
 (segment (start 45.06 86.2) (end 45.0625 90.05) (width 0.24) (layer "F.Cu") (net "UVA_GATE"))
 (segment (start 38.9125 85) (end 40 86.2) (width 0.24) (layer "F.Cu") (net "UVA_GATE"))
 (segment (start 38.9125 82) (end 40 86.2) (width 0.24) (layer "F.Cu") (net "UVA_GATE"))
 (segment (start 40 86.2) (end 45.06 86.2) (width 0.24) (layer "F.Cu") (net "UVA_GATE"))
 (segment (start 62.0625 91) (end 57.5 91) (width 0.24) (layer "F.Cu") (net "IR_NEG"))
 (segment (start 57.5 91) (end 57.5 95.09) (width 0.24) (layer "F.Cu") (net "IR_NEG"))
 (segment (start 46.9375 91) (end 48.5 91) (width 0.24) (layer "F.Cu") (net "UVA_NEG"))
 (segment (start 48.5 91) (end 48.5 95.09) (width 0.24) (layer "F.Cu") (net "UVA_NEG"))
 (segment (start 56.5 88) (end 56.5 95.09) (width 0.24) (layer "F.Cu") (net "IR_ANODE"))
 (segment (start 58 87.4125) (end 56.5 88) (width 0.24) (layer "F.Cu") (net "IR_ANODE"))
 (segment (start 50 87.4125) (end 49.5 89.5) (width 0.24) (layer "F.Cu") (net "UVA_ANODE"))
 (segment (start 49.5 89.5) (end 49.5 95.09) (width 0.24) (layer "F.Cu") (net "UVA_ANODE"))
 (segment (start 50.9125 80) (end 52 80) (width 0.2) (layer "F.Cu") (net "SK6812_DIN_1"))
 (segment (start 54.5 93.6) (end 54.5 95.09) (width 0.2) (layer "F.Cu") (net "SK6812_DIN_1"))
 (via (at 52 80) (size 0.8) (drill 0.4) (layers "F.Cu" "B.Cu") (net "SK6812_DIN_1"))
 (via (at 54.5 93.6) (size 0.8) (drill 0.4) (layers "F.Cu" "B.Cu") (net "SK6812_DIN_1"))
 (segment (start 56.5 86) (end 54.5 86) (width 0.2) (layer "B.Cu") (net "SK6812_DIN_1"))
 (segment (start 54.5 86) (end 54.5 93.6) (width 0.2) (layer "B.Cu") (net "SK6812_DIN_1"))
 (segment (start 52 80) (end 56.5 80) (width 0.2) (layer "B.Cu") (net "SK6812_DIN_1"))
 (segment (start 56.5 80) (end 56.5 86) (width 0.2) (layer "B.Cu") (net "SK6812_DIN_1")))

